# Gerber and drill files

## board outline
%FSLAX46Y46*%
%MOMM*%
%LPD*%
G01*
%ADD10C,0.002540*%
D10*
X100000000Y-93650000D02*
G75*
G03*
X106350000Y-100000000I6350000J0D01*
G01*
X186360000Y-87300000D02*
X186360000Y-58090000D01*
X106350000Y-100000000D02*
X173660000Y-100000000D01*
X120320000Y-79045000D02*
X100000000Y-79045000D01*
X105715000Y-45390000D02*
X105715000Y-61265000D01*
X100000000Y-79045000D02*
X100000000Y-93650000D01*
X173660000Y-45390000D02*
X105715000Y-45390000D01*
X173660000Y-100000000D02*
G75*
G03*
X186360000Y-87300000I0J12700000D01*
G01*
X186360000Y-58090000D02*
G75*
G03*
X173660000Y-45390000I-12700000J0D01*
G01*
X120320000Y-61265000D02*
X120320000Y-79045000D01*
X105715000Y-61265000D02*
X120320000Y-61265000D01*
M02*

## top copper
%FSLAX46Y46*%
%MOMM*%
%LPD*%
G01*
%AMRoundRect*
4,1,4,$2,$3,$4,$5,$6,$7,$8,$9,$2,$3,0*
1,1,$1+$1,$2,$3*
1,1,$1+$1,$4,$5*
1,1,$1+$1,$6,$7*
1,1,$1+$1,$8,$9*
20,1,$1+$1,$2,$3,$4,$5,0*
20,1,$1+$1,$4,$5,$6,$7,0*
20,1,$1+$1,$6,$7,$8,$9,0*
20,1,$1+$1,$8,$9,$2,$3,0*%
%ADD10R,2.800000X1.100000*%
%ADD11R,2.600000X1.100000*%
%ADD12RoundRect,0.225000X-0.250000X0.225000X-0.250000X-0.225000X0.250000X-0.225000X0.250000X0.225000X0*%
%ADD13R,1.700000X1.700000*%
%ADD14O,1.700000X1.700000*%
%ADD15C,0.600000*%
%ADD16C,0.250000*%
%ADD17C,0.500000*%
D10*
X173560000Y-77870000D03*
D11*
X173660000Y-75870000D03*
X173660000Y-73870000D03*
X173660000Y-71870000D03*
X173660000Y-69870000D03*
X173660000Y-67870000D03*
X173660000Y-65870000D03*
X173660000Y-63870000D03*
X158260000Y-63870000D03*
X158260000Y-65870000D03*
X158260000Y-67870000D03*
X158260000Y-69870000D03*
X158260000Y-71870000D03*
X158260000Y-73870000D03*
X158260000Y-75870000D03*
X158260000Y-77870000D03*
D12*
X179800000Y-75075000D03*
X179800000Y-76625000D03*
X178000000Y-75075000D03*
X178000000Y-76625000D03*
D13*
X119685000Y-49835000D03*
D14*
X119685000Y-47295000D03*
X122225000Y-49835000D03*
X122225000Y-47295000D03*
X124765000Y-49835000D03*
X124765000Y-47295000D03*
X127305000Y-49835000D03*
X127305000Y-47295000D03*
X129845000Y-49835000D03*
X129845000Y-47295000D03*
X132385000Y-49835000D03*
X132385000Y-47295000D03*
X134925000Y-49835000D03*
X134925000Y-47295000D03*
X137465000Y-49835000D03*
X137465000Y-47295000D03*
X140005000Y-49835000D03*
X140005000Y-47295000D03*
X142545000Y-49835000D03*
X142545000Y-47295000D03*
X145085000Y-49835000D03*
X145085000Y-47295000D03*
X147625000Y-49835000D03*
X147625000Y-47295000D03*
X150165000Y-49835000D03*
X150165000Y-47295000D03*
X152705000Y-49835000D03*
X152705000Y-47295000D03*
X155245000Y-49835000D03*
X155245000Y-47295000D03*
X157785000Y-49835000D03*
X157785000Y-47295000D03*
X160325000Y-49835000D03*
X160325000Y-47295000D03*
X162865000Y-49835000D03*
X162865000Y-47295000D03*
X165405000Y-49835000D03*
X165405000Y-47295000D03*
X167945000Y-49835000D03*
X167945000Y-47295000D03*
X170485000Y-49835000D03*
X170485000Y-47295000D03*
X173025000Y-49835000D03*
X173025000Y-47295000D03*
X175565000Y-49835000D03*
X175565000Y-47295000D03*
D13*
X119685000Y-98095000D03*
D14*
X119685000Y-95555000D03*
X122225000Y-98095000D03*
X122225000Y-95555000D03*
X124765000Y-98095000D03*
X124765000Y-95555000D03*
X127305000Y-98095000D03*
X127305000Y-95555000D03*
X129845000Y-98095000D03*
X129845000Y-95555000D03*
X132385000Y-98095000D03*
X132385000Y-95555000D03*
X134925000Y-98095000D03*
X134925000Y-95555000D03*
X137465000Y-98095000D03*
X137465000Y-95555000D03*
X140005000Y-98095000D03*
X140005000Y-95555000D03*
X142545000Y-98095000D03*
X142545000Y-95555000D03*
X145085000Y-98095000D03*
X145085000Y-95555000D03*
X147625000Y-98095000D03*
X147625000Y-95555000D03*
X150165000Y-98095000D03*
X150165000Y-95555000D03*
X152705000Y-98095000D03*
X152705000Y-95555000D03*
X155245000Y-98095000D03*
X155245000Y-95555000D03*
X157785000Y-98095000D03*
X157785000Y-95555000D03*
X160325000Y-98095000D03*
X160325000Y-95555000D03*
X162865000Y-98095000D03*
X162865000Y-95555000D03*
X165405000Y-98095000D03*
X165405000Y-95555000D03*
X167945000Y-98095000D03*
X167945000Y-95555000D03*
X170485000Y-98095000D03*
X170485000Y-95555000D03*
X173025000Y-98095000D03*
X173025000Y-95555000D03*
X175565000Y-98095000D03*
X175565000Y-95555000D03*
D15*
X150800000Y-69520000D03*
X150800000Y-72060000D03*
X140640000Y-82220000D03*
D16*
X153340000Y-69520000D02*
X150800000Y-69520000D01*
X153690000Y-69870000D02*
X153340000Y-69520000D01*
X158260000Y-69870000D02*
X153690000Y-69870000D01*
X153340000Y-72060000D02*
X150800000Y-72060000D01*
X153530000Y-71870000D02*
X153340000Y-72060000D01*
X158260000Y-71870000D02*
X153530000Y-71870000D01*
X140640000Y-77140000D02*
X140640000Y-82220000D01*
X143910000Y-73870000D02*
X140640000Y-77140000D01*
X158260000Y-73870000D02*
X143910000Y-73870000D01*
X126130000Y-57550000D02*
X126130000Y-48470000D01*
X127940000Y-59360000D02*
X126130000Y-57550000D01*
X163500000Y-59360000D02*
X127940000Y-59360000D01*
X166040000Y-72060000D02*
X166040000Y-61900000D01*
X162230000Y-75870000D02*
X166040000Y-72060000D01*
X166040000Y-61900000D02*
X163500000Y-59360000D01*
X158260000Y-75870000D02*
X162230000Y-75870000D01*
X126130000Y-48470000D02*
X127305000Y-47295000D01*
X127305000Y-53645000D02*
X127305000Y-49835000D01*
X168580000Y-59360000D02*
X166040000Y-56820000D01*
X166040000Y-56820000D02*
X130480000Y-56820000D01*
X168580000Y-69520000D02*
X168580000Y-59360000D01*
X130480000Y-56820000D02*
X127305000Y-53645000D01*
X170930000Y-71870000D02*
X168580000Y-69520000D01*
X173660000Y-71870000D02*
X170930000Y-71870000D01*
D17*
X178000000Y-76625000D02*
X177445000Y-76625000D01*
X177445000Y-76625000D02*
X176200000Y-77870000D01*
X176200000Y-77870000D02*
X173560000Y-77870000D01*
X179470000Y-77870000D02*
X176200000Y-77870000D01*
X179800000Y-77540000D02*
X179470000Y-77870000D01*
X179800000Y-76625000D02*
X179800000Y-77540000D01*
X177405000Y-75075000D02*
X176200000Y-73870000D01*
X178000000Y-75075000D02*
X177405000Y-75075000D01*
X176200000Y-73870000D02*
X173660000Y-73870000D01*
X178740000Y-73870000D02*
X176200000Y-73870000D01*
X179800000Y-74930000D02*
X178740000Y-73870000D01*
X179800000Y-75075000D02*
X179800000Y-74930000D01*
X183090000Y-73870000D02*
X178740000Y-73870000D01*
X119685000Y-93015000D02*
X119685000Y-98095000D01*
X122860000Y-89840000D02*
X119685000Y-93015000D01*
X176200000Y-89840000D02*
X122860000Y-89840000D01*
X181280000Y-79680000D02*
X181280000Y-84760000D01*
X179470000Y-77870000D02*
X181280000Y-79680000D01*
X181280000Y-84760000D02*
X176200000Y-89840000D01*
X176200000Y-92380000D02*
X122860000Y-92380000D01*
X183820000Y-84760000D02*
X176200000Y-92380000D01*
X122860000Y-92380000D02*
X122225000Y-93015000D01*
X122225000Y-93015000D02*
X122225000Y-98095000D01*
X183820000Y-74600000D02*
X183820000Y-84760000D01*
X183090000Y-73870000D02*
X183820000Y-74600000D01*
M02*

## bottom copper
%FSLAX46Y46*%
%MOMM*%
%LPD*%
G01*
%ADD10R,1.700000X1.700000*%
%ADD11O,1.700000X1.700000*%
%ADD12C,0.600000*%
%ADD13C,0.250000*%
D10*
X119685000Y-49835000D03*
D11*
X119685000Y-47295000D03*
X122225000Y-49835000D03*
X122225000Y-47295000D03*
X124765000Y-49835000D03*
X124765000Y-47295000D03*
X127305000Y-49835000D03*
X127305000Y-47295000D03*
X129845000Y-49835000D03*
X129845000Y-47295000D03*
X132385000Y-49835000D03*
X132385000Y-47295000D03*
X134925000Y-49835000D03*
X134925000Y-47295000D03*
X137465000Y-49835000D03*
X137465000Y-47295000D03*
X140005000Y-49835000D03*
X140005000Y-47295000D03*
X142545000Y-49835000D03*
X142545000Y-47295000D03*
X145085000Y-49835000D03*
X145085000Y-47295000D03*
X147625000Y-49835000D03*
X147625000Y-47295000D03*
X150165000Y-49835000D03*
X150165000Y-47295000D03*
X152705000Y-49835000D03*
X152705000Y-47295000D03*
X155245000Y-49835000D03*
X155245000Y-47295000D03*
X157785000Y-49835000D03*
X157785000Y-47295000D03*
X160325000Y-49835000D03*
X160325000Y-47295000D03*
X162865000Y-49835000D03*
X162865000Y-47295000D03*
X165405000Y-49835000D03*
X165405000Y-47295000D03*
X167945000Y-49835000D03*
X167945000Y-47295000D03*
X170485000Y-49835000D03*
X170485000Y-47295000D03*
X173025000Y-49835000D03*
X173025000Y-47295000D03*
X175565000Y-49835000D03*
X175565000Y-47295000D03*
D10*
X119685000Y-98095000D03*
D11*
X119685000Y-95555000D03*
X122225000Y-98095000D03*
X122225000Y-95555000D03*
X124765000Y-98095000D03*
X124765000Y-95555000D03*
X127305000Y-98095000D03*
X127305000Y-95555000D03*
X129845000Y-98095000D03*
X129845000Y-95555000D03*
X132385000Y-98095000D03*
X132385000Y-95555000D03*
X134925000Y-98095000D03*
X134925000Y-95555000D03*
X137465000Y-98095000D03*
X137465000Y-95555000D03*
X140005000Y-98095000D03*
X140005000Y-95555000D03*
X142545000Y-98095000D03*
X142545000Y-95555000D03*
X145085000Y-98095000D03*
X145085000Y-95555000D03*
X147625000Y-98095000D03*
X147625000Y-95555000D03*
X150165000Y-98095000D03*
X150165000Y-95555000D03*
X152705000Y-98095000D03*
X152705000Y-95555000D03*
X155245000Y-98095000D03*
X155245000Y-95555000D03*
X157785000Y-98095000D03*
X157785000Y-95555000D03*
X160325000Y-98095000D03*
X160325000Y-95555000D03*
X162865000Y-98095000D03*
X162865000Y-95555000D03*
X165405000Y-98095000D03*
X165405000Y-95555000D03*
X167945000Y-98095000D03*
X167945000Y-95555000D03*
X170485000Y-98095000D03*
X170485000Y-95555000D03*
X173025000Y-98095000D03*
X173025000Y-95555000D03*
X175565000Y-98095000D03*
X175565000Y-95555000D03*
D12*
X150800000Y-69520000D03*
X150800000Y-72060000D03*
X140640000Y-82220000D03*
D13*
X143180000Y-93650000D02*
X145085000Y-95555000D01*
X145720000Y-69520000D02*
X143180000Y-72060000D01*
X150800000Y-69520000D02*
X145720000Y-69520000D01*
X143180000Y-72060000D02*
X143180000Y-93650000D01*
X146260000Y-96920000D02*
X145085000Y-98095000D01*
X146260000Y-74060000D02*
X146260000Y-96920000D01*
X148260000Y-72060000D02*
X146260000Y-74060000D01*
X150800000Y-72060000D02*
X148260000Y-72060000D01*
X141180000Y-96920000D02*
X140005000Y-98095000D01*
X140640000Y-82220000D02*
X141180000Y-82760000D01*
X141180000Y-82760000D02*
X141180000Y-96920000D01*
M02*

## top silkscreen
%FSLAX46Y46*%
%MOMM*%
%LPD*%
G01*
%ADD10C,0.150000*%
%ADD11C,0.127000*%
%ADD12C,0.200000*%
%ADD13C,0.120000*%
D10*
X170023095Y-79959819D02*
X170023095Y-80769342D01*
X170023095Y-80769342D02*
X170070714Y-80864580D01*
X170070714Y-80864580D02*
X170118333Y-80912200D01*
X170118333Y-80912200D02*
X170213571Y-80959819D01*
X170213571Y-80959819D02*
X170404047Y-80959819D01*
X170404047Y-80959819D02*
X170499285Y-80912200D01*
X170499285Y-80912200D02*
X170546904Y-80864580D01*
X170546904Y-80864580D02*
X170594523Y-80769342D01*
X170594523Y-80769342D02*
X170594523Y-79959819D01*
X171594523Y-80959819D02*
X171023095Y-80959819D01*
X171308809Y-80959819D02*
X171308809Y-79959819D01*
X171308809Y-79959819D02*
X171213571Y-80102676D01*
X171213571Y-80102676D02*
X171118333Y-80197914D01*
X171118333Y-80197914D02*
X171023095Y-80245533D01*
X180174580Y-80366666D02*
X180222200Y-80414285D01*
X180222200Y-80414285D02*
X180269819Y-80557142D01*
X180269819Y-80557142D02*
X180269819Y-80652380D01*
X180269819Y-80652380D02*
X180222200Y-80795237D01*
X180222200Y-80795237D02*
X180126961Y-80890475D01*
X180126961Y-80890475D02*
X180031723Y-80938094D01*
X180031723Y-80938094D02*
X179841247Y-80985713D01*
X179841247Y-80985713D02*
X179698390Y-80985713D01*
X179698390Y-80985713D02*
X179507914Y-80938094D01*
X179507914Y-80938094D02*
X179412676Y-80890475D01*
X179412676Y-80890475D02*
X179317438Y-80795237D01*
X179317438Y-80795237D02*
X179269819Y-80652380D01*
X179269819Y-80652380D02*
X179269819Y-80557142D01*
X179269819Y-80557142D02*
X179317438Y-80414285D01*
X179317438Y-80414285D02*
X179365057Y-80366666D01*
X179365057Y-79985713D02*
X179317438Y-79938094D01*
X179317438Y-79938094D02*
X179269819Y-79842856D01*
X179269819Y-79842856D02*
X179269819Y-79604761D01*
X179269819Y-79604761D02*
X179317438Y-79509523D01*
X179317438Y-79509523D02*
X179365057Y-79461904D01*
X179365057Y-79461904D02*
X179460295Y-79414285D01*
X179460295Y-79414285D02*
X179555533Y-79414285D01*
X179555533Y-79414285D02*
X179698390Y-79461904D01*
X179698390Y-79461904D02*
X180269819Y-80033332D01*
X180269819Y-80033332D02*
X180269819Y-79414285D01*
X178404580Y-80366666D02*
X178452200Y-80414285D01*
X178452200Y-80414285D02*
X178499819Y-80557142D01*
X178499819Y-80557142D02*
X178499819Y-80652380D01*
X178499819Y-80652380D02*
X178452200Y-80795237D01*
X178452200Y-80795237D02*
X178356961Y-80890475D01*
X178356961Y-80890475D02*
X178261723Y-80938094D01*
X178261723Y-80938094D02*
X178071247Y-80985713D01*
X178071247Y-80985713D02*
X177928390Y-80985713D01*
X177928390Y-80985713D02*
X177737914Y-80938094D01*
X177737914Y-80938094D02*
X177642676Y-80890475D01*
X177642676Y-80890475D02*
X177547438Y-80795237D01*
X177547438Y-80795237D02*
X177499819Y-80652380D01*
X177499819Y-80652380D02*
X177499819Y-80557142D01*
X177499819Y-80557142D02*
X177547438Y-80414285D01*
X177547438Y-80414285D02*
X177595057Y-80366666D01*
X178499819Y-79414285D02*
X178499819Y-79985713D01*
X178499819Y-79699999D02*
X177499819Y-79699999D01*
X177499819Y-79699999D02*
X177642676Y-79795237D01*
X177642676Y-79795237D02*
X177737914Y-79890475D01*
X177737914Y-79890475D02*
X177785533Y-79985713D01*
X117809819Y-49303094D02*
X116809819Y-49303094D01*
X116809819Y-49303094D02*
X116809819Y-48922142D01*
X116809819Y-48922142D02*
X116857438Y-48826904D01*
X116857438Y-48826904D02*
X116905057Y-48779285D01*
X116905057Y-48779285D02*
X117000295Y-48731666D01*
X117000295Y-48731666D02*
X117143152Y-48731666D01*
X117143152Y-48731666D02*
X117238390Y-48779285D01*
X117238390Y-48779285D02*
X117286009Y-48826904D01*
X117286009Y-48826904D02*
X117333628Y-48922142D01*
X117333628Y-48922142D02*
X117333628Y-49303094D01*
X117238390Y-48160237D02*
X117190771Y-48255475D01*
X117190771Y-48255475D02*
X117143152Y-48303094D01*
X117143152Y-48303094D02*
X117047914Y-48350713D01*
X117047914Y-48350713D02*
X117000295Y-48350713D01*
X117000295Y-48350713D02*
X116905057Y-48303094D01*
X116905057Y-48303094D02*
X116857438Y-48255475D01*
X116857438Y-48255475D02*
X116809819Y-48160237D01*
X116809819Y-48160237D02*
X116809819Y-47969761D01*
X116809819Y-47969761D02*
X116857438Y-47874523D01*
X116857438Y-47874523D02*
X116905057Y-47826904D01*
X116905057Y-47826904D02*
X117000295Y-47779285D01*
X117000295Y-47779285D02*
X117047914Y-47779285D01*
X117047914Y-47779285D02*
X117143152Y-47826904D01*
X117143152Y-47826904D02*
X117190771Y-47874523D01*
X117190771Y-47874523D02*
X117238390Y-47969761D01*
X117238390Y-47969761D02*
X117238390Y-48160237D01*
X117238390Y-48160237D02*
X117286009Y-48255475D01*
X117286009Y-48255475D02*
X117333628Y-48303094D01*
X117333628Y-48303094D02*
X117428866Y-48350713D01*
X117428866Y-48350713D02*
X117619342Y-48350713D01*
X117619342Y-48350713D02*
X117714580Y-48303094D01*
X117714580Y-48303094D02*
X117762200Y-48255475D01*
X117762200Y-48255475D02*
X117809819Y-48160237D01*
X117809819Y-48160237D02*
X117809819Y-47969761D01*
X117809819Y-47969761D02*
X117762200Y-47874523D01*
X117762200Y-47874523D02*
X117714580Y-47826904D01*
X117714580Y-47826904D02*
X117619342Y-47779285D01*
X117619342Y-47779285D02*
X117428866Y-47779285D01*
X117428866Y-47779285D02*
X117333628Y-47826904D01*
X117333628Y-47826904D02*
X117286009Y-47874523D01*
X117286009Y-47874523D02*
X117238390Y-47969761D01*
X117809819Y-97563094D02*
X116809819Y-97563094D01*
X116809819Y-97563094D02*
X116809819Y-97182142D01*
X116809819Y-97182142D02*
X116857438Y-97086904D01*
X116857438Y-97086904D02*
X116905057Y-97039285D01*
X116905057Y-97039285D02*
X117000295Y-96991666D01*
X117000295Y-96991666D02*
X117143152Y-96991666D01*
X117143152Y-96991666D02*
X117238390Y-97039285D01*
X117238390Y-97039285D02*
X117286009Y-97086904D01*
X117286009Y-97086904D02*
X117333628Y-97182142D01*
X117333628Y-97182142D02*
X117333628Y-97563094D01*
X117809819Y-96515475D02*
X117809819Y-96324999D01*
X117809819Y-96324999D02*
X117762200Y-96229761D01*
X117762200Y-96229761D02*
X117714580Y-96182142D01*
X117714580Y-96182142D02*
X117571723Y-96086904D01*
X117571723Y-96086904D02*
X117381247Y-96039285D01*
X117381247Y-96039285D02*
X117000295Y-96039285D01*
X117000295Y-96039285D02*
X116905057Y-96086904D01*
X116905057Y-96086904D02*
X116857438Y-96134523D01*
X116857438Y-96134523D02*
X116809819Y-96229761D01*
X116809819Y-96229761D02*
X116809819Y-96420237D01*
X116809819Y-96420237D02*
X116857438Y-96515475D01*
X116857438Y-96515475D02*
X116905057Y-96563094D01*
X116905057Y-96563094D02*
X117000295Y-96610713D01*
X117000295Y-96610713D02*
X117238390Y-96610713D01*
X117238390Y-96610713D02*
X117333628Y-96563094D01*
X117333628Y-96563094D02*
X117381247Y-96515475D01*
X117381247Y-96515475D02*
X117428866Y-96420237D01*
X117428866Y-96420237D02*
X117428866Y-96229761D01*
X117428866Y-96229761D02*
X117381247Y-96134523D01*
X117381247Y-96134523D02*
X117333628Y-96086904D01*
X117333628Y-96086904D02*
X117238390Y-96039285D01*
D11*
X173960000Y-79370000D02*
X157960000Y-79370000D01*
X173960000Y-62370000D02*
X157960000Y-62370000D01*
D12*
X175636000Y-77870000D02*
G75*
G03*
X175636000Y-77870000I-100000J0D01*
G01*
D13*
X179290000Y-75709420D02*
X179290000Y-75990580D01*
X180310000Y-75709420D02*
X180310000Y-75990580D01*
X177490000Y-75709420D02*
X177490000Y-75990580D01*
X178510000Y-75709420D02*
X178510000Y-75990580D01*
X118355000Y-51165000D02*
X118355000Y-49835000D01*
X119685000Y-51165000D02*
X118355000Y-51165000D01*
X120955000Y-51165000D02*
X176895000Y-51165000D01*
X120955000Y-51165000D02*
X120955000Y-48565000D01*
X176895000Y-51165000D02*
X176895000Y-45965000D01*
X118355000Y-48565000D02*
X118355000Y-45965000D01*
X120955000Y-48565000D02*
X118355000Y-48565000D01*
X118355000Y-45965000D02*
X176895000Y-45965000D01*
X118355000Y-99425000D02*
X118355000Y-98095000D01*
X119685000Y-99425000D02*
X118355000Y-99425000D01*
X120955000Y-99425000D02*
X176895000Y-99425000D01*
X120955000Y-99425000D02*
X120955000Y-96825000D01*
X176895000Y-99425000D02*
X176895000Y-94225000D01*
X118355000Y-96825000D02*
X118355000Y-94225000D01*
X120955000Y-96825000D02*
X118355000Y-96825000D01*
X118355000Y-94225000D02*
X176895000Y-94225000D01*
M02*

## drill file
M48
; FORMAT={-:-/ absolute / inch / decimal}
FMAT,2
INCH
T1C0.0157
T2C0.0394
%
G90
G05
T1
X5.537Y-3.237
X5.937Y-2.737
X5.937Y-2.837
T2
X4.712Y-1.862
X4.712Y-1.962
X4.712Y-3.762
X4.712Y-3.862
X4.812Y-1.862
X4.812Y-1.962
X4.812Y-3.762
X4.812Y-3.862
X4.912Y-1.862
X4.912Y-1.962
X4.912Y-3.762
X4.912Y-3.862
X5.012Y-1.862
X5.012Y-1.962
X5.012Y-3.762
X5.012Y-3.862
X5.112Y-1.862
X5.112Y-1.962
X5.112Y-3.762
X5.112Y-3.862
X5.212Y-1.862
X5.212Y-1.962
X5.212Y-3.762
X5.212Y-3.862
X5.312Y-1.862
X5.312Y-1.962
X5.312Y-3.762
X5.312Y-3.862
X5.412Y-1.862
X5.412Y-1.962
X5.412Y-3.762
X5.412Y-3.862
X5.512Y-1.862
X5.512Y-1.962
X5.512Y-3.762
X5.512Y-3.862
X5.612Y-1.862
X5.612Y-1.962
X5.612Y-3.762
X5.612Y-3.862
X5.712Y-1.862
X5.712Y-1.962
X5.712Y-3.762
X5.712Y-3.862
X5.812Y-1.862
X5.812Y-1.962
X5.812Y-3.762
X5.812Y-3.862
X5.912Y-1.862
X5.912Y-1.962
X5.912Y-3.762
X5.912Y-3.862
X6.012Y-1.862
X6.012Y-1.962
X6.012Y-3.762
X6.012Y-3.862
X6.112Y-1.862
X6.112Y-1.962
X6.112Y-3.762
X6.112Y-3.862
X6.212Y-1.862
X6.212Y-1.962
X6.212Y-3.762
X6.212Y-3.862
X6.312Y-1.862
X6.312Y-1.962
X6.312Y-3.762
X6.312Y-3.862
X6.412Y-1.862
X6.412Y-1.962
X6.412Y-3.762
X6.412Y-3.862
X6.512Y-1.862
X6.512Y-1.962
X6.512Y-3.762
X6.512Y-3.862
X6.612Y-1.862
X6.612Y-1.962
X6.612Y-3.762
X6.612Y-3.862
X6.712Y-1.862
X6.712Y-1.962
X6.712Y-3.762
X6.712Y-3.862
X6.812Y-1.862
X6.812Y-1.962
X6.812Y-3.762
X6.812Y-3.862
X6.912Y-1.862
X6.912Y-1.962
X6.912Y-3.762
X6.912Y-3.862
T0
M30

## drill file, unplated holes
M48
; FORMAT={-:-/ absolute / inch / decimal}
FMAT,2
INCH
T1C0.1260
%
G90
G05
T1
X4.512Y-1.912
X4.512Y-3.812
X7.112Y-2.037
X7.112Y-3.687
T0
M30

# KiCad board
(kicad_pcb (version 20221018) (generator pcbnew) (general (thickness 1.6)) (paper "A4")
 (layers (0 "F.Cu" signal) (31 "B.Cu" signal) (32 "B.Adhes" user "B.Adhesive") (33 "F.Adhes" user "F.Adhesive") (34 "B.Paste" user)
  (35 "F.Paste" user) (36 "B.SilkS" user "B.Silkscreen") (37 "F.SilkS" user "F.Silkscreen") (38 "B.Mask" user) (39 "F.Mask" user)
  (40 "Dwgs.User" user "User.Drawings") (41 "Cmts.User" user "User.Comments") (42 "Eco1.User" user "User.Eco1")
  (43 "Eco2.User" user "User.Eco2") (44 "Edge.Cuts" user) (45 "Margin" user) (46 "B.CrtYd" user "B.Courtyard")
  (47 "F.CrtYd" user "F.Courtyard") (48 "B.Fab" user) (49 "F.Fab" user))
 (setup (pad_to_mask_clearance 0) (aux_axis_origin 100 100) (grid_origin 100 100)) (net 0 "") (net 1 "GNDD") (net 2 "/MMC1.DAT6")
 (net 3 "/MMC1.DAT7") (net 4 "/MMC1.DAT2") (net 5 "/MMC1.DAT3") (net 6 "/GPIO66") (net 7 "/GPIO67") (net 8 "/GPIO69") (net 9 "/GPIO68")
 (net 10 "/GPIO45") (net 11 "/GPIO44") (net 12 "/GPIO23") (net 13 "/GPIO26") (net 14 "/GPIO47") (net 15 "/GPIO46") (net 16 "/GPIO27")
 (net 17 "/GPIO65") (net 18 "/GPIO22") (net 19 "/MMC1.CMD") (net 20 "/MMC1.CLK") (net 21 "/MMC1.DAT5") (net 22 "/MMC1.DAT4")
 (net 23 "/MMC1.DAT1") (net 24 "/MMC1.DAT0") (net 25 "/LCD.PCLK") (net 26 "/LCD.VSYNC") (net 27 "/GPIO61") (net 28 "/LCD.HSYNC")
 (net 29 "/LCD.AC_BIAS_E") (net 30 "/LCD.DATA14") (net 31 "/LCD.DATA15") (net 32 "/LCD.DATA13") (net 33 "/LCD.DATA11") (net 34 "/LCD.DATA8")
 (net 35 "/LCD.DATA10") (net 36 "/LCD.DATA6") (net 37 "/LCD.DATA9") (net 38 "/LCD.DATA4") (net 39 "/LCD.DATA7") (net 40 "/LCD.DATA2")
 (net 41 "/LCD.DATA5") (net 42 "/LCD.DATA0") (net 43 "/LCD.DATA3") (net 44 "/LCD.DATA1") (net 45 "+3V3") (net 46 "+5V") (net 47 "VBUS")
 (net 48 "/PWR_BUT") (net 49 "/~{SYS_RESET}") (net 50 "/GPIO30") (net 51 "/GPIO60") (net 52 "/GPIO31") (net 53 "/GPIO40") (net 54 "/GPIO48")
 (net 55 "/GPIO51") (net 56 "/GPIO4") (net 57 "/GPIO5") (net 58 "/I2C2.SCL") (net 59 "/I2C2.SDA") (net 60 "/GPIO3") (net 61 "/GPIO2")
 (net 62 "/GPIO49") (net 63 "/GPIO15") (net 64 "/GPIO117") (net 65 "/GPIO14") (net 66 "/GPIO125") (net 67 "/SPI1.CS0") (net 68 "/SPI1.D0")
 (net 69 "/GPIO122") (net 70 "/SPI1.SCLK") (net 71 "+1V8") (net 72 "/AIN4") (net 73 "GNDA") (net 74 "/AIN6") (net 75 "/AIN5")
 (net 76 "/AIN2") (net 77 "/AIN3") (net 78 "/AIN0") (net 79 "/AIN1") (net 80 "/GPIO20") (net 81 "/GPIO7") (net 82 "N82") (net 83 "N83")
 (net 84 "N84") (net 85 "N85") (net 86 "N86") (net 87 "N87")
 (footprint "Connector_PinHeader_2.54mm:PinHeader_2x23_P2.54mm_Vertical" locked (layer "F.Cu") (at 119.685 49.835 90)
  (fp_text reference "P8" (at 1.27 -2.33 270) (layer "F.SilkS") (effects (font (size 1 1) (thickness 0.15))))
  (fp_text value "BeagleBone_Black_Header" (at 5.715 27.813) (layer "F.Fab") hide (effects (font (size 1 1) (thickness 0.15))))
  (fp_line (start -1.33 -1.33) (end 0 -1.33) (stroke (width 0.12) (type solid)) (layer "F.SilkS"))
  (fp_line (start -1.33 0) (end -1.33 -1.33) (stroke (width 0.12) (type solid)) (layer "F.SilkS"))
  (fp_line (start -1.33 1.27) (end -1.33 57.21) (stroke (width 0.12) (type solid)) (layer "F.SilkS"))
  (fp_line (start -1.33 1.27) (end 1.27 1.27) (stroke (width 0.12) (type solid)) (layer "F.SilkS"))
  (fp_line (start -1.33 57.21) (end 3.87 57.21) (stroke (width 0.12) (type solid)) (layer "F.SilkS"))
  (fp_line (start 1.27 -1.33) (end 3.87 -1.33) (stroke (width 0.12) (type solid)) (layer "F.SilkS"))
  (fp_line (start 1.27 1.27) (end 1.27 -1.33) (stroke (width 0.12) (type solid)) (layer "F.SilkS"))
  (fp_line (start 3.87 -1.33) (end 3.87 57.21) (stroke (width 0.12) (type solid)) (layer "F.SilkS"))
  (pad "1" thru_hole rect locked (at 0 0 90) (size 1.7 1.7) (drill 1) (layers "*.Cu" "*.Mask") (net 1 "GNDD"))
  (pad "2" thru_hole oval locked (at 2.54 0 90) (size 1.7 1.7) (drill 1) (layers "*.Cu" "*.Mask") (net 1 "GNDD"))
  (pad "3" thru_hole oval locked (at 0 2.54 90) (size 1.7 1.7) (drill 1) (layers "*.Cu" "*.Mask") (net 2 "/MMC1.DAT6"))
  (pad "4" thru_hole oval locked (at 2.54 2.54 90) (size 1.7 1.7) (drill 1) (layers "*.Cu" "*.Mask") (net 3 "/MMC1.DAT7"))
  (pad "5" thru_hole oval locked (at 0 5.08 90) (size 1.7 1.7) (drill 1) (layers "*.Cu" "*.Mask") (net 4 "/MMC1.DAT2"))
  (pad "6" thru_hole oval locked (at 2.54 5.08 90) (size 1.7 1.7) (drill 1) (layers "*.Cu" "*.Mask") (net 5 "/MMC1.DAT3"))
  (pad "7" thru_hole oval locked (at 0 7.62 90) (size 1.7 1.7) (drill 1) (layers "*.Cu" "*.Mask") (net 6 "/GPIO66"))
  (pad "8" thru_hole oval locked (at 2.54 7.62 90) (size 1.7 1.7) (drill 1) (layers "*.Cu" "*.Mask") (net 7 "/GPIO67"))
  (pad "9" thru_hole oval locked (at 0 10.16 90) (size 1.7 1.7) (drill 1) (layers "*.Cu" "*.Mask") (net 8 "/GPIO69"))
  (pad "10" thru_hole oval locked (at 2.54 10.16 90) (size 1.7 1.7) (drill 1) (layers "*.Cu" "*.Mask") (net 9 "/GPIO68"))
  (pad "11" thru_hole oval locked (at 0 12.7 90) (size 1.7 1.7) (drill 1) (layers "*.Cu" "*.Mask") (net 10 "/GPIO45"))
  (pad "12" thru_hole oval locked (at 2.54 12.7 90) (size 1.7 1.7) (drill 1) (layers "*.Cu" "*.Mask") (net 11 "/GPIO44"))
  (pad "13" thru_hole oval locked (at 0 15.24 90) (size 1.7 1.7) (drill 1) (layers "*.Cu" "*.Mask") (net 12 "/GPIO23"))
  (pad "14" thru_hole oval locked (at 2.54 15.24 90) (size 1.7 1.7) (drill 1) (layers "*.Cu" "*.Mask") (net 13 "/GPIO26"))
  (pad "15" thru_hole oval locked (at 0 17.78 90) (size 1.7 1.7) (drill 1) (layers "*.Cu" "*.Mask") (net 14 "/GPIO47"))
  (pad "16" thru_hole oval locked (at 2.54 17.78 90) (size 1.7 1.7) (drill 1) (layers "*.Cu" "*.Mask") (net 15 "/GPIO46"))
  (pad "17" thru_hole oval locked (at 0 20.32 90) (size 1.7 1.7) (drill 1) (layers "*.Cu" "*.Mask") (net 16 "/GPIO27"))
  (pad "18" thru_hole oval locked (at 2.54 20.32 90) (size 1.7 1.7) (drill 1) (layers "*.Cu" "*.Mask") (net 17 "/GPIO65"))
  (pad "19" thru_hole oval locked (at 0 22.86 90) (size 1.7 1.7) (drill 1) (layers "*.Cu" "*.Mask") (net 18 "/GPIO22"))
  (pad "20" thru_hole oval locked (at 2.54 22.86 90) (size 1.7 1.7) (drill 1) (layers "*.Cu" "*.Mask") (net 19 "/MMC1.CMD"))
  (pad "21" thru_hole oval locked (at 0 25.4 90) (size 1.7 1.7) (drill 1) (layers "*.Cu" "*.Mask") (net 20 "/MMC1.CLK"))
  (pad "22" thru_hole oval locked (at 2.54 25.4 90) (size 1.7 1.7) (drill 1) (layers "*.Cu" "*.Mask") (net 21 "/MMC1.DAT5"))
  (pad "23" thru_hole oval locked (at 0 27.94 90) (size 1.7 1.7) (drill 1) (layers "*.Cu" "*.Mask") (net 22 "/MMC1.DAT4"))
  (pad "24" thru_hole oval locked (at 2.54 27.94 90) (size 1.7 1.7) (drill 1) (layers "*.Cu" "*.Mask") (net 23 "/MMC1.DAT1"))
  (pad "25" thru_hole oval locked (at 0 30.48 90) (size 1.7 1.7) (drill 1) (layers "*.Cu" "*.Mask") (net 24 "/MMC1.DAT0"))
  (pad "26" thru_hole oval locked (at 2.54 30.48 90) (size 1.7 1.7) (drill 1) (layers "*.Cu" "*.Mask") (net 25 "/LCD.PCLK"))
  (pad "27" thru_hole oval locked (at 0 33.02 90) (size 1.7 1.7) (drill 1) (layers "*.Cu" "*.Mask") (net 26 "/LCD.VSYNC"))
  (pad "28" thru_hole oval locked (at 2.54 33.02 90) (size 1.7 1.7) (drill 1) (layers "*.Cu" "*.Mask") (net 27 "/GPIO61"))
  (pad "29" thru_hole oval locked (at 0 35.56 90) (size 1.7 1.7) (drill 1) (layers "*.Cu" "*.Mask") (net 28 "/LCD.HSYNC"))
  (pad "30" thru_hole oval locked (at 2.54 35.56 90) (size 1.7 1.7) (drill 1) (layers "*.Cu" "*.Mask") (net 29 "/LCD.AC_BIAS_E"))
  (pad "31" thru_hole oval locked (at 0 38.1 90) (size 1.7 1.7) (drill 1) (layers "*.Cu" "*.Mask") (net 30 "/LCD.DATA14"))
  (pad "32" thru_hole oval locked (at 2.54 38.1 90) (size 1.7 1.7) (drill 1) (layers "*.Cu" "*.Mask") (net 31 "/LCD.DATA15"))
  (pad "33" thru_hole oval locked (at 0 40.64 90) (size 1.7 1.7) (drill 1) (layers "*.Cu" "*.Mask") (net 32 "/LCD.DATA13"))
  (pad "34" thru_hole oval locked (at 2.54 40.64 90) (size 1.7 1.7) (drill 1) (layers "*.Cu" "*.Mask") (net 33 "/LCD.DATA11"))
  (pad "35" thru_hole oval locked (at 0 43.18 90) (size 1.7 1.7) (drill 1) (layers "*.Cu" "*.Mask") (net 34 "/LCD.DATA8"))
  (pad "36" thru_hole oval locked (at 2.54 43.18 90) (size 1.7 1.7) (drill 1) (layers "*.Cu" "*.Mask") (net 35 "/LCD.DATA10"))
  (pad "37" thru_hole oval locked (at 0 45.72 90) (size 1.7 1.7) (drill 1) (layers "*.Cu" "*.Mask") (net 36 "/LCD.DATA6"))
  (pad "38" thru_hole oval locked (at 2.54 45.72 90) (size 1.7 1.7) (drill 1) (layers "*.Cu" "*.Mask") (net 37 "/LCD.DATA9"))
  (pad "39" thru_hole oval locked (at 0 48.26 90) (size 1.7 1.7) (drill 1) (layers "*.Cu" "*.Mask") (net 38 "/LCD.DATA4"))
  (pad "40" thru_hole oval locked (at 2.54 48.26 90) (size 1.7 1.7) (drill 1) (layers "*.Cu" "*.Mask") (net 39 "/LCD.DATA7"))
  (pad "41" thru_hole oval locked (at 0 50.8 90) (size 1.7 1.7) (drill 1) (layers "*.Cu" "*.Mask") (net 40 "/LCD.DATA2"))
  (pad "42" thru_hole oval locked (at 2.54 50.8 90) (size 1.7 1.7) (drill 1) (layers "*.Cu" "*.Mask") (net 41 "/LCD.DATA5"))
  (pad "43" thru_hole oval locked (at 0 53.34 90) (size 1.7 1.7) (drill 1) (layers "*.Cu" "*.Mask") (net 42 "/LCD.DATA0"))
  (pad "44" thru_hole oval locked (at 2.54 53.34 90) (size 1.7 1.7) (drill 1) (layers "*.Cu" "*.Mask") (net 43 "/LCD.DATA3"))
  (pad "45" thru_hole oval locked (at 0 55.88 90) (size 1.7 1.7) (drill 1) (layers "*.Cu" "*.Mask") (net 1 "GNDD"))
  (pad "46" thru_hole oval locked (at 2.54 55.88 90) (size 1.7 1.7) (drill 1) (layers "*.Cu" "*.Mask") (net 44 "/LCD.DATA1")))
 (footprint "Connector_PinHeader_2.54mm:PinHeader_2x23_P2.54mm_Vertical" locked (layer "F.Cu") (at 119.685 98.095 90)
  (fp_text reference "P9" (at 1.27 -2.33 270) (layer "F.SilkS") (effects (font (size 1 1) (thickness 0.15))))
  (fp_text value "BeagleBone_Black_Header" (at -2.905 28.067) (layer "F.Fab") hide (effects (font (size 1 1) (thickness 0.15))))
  (fp_line (start -1.33 -1.33) (end 0 -1.33) (stroke (width 0.12) (type solid)) (layer "F.SilkS"))
  (fp_line (start -1.33 0) (end -1.33 -1.33) (stroke (width 0.12) (type solid)) (layer "F.SilkS"))
  (fp_line (start -1.33 1.27) (end -1.33 57.21) (stroke (width 0.12) (type solid)) (layer "F.SilkS"))
  (fp_line (start -1.33 1.27) (end 1.27 1.27) (stroke (width 0.12) (type solid)) (layer "F.SilkS"))
  (fp_line (start -1.33 57.21) (end 3.87 57.21) (stroke (width 0.12) (type solid)) (layer "F.SilkS"))
  (fp_line (start 1.27 -1.33) (end 3.87 -1.33) (stroke (width 0.12) (type solid)) (layer "F.SilkS"))
  (fp_line (start 1.27 1.27) (end 1.27 -1.33) (stroke (width 0.12) (type solid)) (layer "F.SilkS"))
  (fp_line (start 3.87 -1.33) (end 3.87 57.21) (stroke (width 0.12) (type solid)) (layer "F.SilkS"))
  (pad "1" thru_hole rect locked (at 0 0 90) (size 1.7 1.7) (drill 1) (layers "*.Cu" "*.Mask") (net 1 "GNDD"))
  (pad "2" thru_hole oval locked (at 2.54 0 90) (size 1.7 1.7) (drill 1) (layers "*.Cu" "*.Mask") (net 1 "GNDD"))
  (pad "3" thru_hole oval locked (at 0 2.54 90) (size 1.7 1.7) (drill 1) (layers "*.Cu" "*.Mask") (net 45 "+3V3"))
  (pad "4" thru_hole oval locked (at 2.54 2.54 90) (size 1.7 1.7) (drill 1) (layers "*.Cu" "*.Mask") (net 45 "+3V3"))
  (pad "5" thru_hole oval locked (at 0 5.08 90) (size 1.7 1.7) (drill 1) (layers "*.Cu" "*.Mask") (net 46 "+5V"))
  (pad "6" thru_hole oval locked (at 2.54 5.08 90) (size 1.7 1.7) (drill 1) (layers "*.Cu" "*.Mask") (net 46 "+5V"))
  (pad "7" thru_hole oval locked (at 0 7.62 90) (size 1.7 1.7) (drill 1) (layers "*.Cu" "*.Mask") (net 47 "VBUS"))
  (pad "8" thru_hole oval locked (at 2.54 7.62 90) (size 1.7 1.7) (drill 1) (layers "*.Cu" "*.Mask") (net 47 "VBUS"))
  (pad "9" thru_hole oval locked (at 0 10.16 90) (size 1.7 1.7) (drill 1) (layers "*.Cu" "*.Mask") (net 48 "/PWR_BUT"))
  (pad "10" thru_hole oval locked (at 2.54 10.16 90) (size 1.7 1.7) (drill 1) (layers "*.Cu" "*.Mask") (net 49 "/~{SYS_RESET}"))
  (pad "11" thru_hole oval locked (at 0 12.7 90) (size 1.7 1.7) (drill 1) (layers "*.Cu" "*.Mask") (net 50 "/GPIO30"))
  (pad "12" thru_hole oval locked (at 2.54 12.7 90) (size 1.7 1.7) (drill 1) (layers "*.Cu" "*.Mask") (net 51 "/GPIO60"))
  (pad "13" thru_hole oval locked (at 0 15.24 90) (size 1.7 1.7) (drill 1) (layers "*.Cu" "*.Mask") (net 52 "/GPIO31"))
  (pad "14" thru_hole oval locked (at 2.54 15.24 90) (size 1.7 1.7) (drill 1) (layers "*.Cu" "*.Mask") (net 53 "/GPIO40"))
  (pad "15" thru_hole oval locked (at 0 17.78 90) (size 1.7 1.7) (drill 1) (layers "*.Cu" "*.Mask") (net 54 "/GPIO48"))
  (pad "16" thru_hole oval locked (at 2.54 17.78 90) (size 1.7 1.7) (drill 1) (layers "*.Cu" "*.Mask") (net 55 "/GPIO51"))
  (pad "17" thru_hole oval locked (at 0 20.32 90) (size 1.7 1.7) (drill 1) (layers "*.Cu" "*.Mask") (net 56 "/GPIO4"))
  (pad "18" thru_hole oval locked (at 2.54 20.32 90) (size 1.7 1.7) (drill 1) (layers "*.Cu" "*.Mask") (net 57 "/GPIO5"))
  (pad "19" thru_hole oval locked (at 0 22.86 90) (size 1.7 1.7) (drill 1) (layers "*.Cu" "*.Mask") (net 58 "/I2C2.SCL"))
  (pad "20" thru_hole oval locked (at 2.54 22.86 90) (size 1.7 1.7) (drill 1) (layers "*.Cu" "*.Mask") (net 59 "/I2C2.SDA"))
  (pad "21" thru_hole oval locked (at 0 25.4 90) (size 1.7 1.7) (drill 1) (layers "*.Cu" "*.Mask") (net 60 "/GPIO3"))
  (pad "22" thru_hole oval locked (at 2.54 25.4 90) (size 1.7 1.7) (drill 1) (layers "*.Cu" "*.Mask") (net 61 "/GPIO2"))
  (pad "23" thru_hole oval locked (at 0 27.94 90) (size 1.7 1.7) (drill 1) (layers "*.Cu" "*.Mask") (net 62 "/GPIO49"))
  (pad "24" thru_hole oval locked (at 2.54 27.94 90) (size 1.7 1.7) (drill 1) (layers "*.Cu" "*.Mask") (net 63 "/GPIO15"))
  (pad "25" thru_hole oval locked (at 0 30.48 90) (size 1.7 1.7) (drill 1) (layers "*.Cu" "*.Mask") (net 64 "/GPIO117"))
  (pad "26" thru_hole oval locked (at 2.54 30.48 90) (size 1.7 1.7) (drill 1) (layers "*.Cu" "*.Mask") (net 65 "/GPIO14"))
  (pad "27" thru_hole oval locked (at 0 33.02 90) (size 1.7 1.7) (drill 1) (layers "*.Cu" "*.Mask") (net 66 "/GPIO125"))
  (pad "28" thru_hole oval locked (at 2.54 33.02 90) (size 1.7 1.7) (drill 1) (layers "*.Cu" "*.Mask") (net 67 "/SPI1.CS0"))
  (pad "29" thru_hole oval locked (at 0 35.56 90) (size 1.7 1.7) (drill 1) (layers "*.Cu" "*.Mask") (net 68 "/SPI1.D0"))
  (pad "30" thru_hole oval locked (at 2.54 35.56 90) (size 1.7 1.7) (drill 1) (layers "*.Cu" "*.Mask") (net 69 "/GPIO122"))
  (pad "31" thru_hole oval locked (at 0 38.1 90) (size 1.7 1.7) (drill 1) (layers "*.Cu" "*.Mask") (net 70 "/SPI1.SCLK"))
  (pad "32" thru_hole oval locked (at 2.54 38.1 90) (size 1.7 1.7) (drill 1) (layers "*.Cu" "*.Mask") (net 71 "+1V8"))
  (pad "33" thru_hole oval locked (at 0 40.64 90) (size 1.7 1.7) (drill 1) (layers "*.Cu" "*.Mask") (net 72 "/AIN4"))
  (pad "34" thru_hole oval locked (at 2.54 40.64 90) (size 1.7 1.7) (drill 1) (layers "*.Cu" "*.Mask") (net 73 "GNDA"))
  (pad "35" thru_hole oval locked (at 0 43.18 90) (size 1.7 1.7) (drill 1) (layers "*.Cu" "*.Mask") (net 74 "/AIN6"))
  (pad "36" thru_hole oval locked (at 2.54 43.18 90) (size 1.7 1.7) (drill 1) (layers "*.Cu" "*.Mask") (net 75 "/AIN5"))
  (pad "37" thru_hole oval locked (at 0 45.72 90) (size 1.7 1.7) (drill 1) (layers "*.Cu" "*.Mask") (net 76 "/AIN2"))
  (pad "38" thru_hole oval locked (at 2.54 45.72 90) (size 1.7 1.7) (drill 1) (layers "*.Cu" "*.Mask") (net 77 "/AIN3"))
  (pad "39" thru_hole oval locked (at 0 48.26 90) (size 1.7 1.7) (drill 1) (layers "*.Cu" "*.Mask") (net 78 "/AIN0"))
  (pad "40" thru_hole oval locked (at 2.54 48.26 90) (size 1.7 1.7) (drill 1) (layers "*.Cu" "*.Mask") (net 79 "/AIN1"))
  (pad "41" thru_hole oval locked (at 0 50.8 90) (size 1.7 1.7) (drill 1) (layers "*.Cu" "*.Mask") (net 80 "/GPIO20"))
  (pad "42" thru_hole oval locked (at 2.54 50.8 90) (size 1.7 1.7) (drill 1) (layers "*.Cu" "*.Mask") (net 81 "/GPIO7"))
  (pad "43" thru_hole oval locked (at 0 53.34 90) (size 1.7 1.7) (drill 1) (layers "*.Cu" "*.Mask") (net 1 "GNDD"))
  (pad "44" thru_hole oval locked (at 2.54 53.34 90) (size 1.7 1.7) (drill 1) (layers "*.Cu" "*.Mask") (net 1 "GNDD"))
  (pad "45" thru_hole oval locked (at 0 55.88 90) (size 1.7 1.7) (drill 1) (layers "*.Cu" "*.Mask") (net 1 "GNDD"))
  (pad "46" thru_hole oval locked (at 2.54 55.88 90) (size 1.7 1.7) (drill 1) (layers "*.Cu" "*.Mask") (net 1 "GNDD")))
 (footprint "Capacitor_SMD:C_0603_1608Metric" (layer "F.Cu") (at 178 75.85 -90)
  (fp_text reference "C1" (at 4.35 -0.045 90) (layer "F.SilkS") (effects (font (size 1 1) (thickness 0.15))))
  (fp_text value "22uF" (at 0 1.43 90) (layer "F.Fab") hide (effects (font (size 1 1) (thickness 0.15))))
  (fp_line (start -0.14058 -0.51) (end 0.14058 -0.51) (stroke (width 0.12) (type solid)) (layer "F.SilkS"))
  (fp_line (start -0.14058 0.51) (end 0.14058 0.51) (stroke (width 0.12) (type solid)) (layer "F.SilkS"))
  (pad "1" smd roundrect (at -0.775 0 270) (size 0.9 0.95) (layers "F.Cu" "F.Paste" "F.Mask") (roundrect_rratio 0.25) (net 45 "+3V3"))
  (pad "2" smd roundrect (at 0.775 0 270) (size 0.9 0.95) (layers "F.Cu" "F.Paste" "F.Mask") (roundrect_rratio 0.25) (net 1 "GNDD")))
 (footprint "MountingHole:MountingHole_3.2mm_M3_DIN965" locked (layer "F.Cu") (at 180.645 51.74)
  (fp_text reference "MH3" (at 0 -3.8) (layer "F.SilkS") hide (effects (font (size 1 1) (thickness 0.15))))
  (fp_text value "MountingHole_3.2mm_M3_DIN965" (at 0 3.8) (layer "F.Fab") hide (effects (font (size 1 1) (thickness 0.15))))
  (pad "" np_thru_hole circle locked (at 0 0) (size 3.2 3.2) (drill 3.2) (layers "*.Cu" "*.Mask")))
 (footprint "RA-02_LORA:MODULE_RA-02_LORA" (layer "F.Cu") (at 165.96 70.87 180)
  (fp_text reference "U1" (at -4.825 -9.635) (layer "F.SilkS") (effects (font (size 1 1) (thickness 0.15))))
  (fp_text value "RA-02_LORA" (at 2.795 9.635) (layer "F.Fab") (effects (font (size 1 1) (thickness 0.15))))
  (fp_line (start -8 -8.5) (end 8 -8.5) (stroke (width 0.127) (type solid)) (layer "F.SilkS"))
  (fp_line (start -8 8.5) (end 8 8.5) (stroke (width 0.127) (type solid)) (layer "F.SilkS"))
  (fp_circle (center -9.576 -7) (end -9.476 -7) (stroke (width 0.2) (type solid)) (fill none) (layer "F.SilkS"))
  (pad "1" smd rect (at -7.6 -7 180) (size 2.8 1.1) (layers "F.Cu" "F.Paste" "F.Mask") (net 1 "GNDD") (solder_mask_margin 0.102))
  (pad "2" smd rect (at -7.7 -5 180) (size 2.6 1.1) (layers "F.Cu" "F.Paste" "F.Mask") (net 1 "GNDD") (solder_mask_margin 0.102))
  (pad "3" smd rect (at -7.7 -3 180) (size 2.6 1.1) (layers "F.Cu" "F.Paste" "F.Mask") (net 45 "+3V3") (solder_mask_margin 0.102))
  (pad "4" smd rect (at -7.7 -1 180) (size 2.6 1.1) (layers "F.Cu" "F.Paste" "F.Mask") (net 6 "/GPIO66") (solder_mask_margin 0.102))
  (pad "5" smd rect (at -7.7 1 180) (size 2.6 1.1) (layers "F.Cu" "F.Paste" "F.Mask") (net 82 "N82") (solder_mask_margin 0.102))
  (pad "6" smd rect (at -7.7 3 180) (size 2.6 1.1) (layers "F.Cu" "F.Paste" "F.Mask") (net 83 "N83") (solder_mask_margin 0.102))
  (pad "7" smd rect (at -7.7 5 180) (size 2.6 1.1) (layers "F.Cu" "F.Paste" "F.Mask") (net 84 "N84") (solder_mask_margin 0.102))
  (pad "8" smd rect (at -7.7 7 180) (size 2.6 1.1) (layers "F.Cu" "F.Paste" "F.Mask") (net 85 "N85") (solder_mask_margin 0.102))
  (pad "9" smd rect (at 7.7 7) (size 2.6 1.1) (layers "F.Cu" "F.Paste" "F.Mask") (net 1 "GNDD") (solder_mask_margin 0.102))
  (pad "10" smd rect (at 7.7 5) (size 2.6 1.1) (layers "F.Cu" "F.Paste" "F.Mask") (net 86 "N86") (solder_mask_margin 0.102))
  (pad "11" smd rect (at 7.7 3) (size 2.6 1.1) (layers "F.Cu" "F.Paste" "F.Mask") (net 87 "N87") (solder_mask_margin 0.102))
  (pad "12" smd rect (at 7.7 1) (size 2.6 1.1) (layers "F.Cu" "F.Paste" "F.Mask") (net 61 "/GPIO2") (solder_mask_margin 0.102))
  (pad "13" smd rect (at 7.7 -1) (size 2.6 1.1) (layers "F.Cu" "F.Paste" "F.Mask") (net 60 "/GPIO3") (solder_mask_margin 0.102))
  (pad "14" smd rect (at 7.7 -3) (size 2.6 1.1) (layers "F.Cu" "F.Paste" "F.Mask") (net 56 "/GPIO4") (solder_mask_margin 0.102))
  (pad "15" smd rect (at 7.7 -5) (size 2.6 1.1) (layers "F.Cu" "F.Paste" "F.Mask") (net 7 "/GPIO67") (solder_mask_margin 0.102))
  (pad "16" smd rect (at 7.7 -7) (size 2.6 1.1) (layers "F.Cu" "F.Paste" "F.Mask") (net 1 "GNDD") (solder_mask_margin 0.102)))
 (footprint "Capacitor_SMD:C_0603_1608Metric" (layer "F.Cu") (at 179.8 75.85 -90)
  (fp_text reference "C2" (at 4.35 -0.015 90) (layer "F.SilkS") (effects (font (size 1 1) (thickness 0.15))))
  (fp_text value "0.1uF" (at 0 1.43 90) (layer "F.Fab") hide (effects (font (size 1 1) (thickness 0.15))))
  (fp_line (start -0.14058 -0.51) (end 0.14058 -0.51) (stroke (width 0.12) (type solid)) (layer "F.SilkS"))
  (fp_line (start -0.14058 0.51) (end 0.14058 0.51) (stroke (width 0.12) (type solid)) (layer "F.SilkS"))
  (pad "1" smd roundrect (at -0.775 0 270) (size 0.9 0.95) (layers "F.Cu" "F.Paste" "F.Mask") (roundrect_rratio 0.25) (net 45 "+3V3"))
  (pad "2" smd roundrect (at 0.775 0 270) (size 0.9 0.95) (layers "F.Cu" "F.Paste" "F.Mask") (roundrect_rratio 0.25) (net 1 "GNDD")))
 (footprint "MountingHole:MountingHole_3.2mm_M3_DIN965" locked (layer "F.Cu") (at 180.645 93.65)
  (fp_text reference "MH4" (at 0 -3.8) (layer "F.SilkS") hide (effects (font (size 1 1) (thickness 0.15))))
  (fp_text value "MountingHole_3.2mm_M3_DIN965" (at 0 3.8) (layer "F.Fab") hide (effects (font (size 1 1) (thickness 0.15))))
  (pad "" np_thru_hole circle locked (at 0 0) (size 3.2 3.2) (drill 3.2) (layers "*.Cu" "*.Mask")))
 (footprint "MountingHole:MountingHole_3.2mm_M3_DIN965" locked (layer "F.Cu") (at 114.605 48.565)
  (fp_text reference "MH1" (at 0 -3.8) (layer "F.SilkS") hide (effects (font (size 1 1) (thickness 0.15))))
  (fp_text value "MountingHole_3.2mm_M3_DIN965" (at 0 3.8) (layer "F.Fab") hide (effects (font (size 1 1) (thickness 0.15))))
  (pad "" np_thru_hole circle locked (at 0 0) (size 3.2 3.2) (drill 3.2) (layers "*.Cu" "*.Mask")))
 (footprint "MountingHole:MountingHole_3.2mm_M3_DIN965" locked (layer "F.Cu") (at 114.605 96.825)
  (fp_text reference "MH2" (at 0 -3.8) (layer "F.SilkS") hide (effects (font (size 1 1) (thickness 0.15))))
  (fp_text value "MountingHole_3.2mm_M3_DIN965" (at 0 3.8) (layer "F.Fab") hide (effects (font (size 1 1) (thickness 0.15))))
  (pad "" np_thru_hole circle locked (at 0 0) (size 3.2 3.2) (drill 3.2) (layers "*.Cu" "*.Mask")))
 (gr_arc locked (start 106.35 100) (mid 101.859872 98.140128) (end 100 93.65) (stroke (width 0.00254) (type solid)) (layer "Edge.Cuts"))
 (gr_line locked (start 186.36 87.3) (end 186.36 58.09) (stroke (width 0.00254) (type solid)) (layer "Edge.Cuts"))
 (gr_line locked (start 106.35 100) (end 173.66 100) (stroke (width 0.00254) (type solid)) (layer "Edge.Cuts"))
 (gr_line locked (start 120.32 79.045) (end 100 79.045) (stroke (width 0.00254) (type solid)) (layer "Edge.Cuts"))
 (gr_line locked (start 105.715 45.39) (end 105.715 61.265) (stroke (width 0.00254) (type solid)) (layer "Edge.Cuts"))
 (gr_line locked (start 100 79.045) (end 100 93.65) (stroke (width 0.00254) (type solid)) (layer "Edge.Cuts"))
 (gr_line locked (start 173.66 45.39) (end 105.715 45.39) (stroke (width 0.00254) (type solid)) (layer "Edge.Cuts"))
 (gr_arc locked (start 186.36 87.3) (mid 182.640256 96.280256) (end 173.66 100) (stroke (width 0.00254) (type solid)) (layer "Edge.Cuts"))
 (gr_arc locked (start 173.66 45.39) (mid 182.640256 49.109744) (end 186.36 58.09) (stroke (width 0.00254) (type solid)) (layer "Edge.Cuts"))
 (gr_line locked (start 120.32 61.265) (end 120.32 79.045) (stroke (width 0.00254) (type solid)) (layer "Edge.Cuts"))
 (gr_line locked (start 105.715 61.265) (end 120.32 61.265) (stroke (width 0.00254) (type solid)) (layer "Edge.Cuts"))
 (segment (start 130.48 56.82) (end 127.305 53.645) (width 0.25) (layer "F.Cu") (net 6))
 (segment (start 168.58 69.52) (end 168.58 59.36) (width 0.25) (layer "F.Cu") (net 6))
 (segment (start 166.04 56.82) (end 130.48 56.82) (width 0.25) (layer "F.Cu") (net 6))
 (segment (start 168.58 59.36) (end 166.04 56.82) (width 0.25) (layer "F.Cu") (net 6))
 (segment (start 170.93 71.87) (end 168.58 69.52) (width 0.25) (layer "F.Cu") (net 6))
 (segment (start 173.66 71.87) (end 170.93 71.87) (width 0.25) (layer "F.Cu") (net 6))
 (segment (start 127.305 53.645) (end 127.305 49.835) (width 0.25) (layer "F.Cu") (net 6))
 (segment (start 126.13 57.55) (end 126.13 48.47) (width 0.25) (layer "F.Cu") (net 7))
 (segment (start 166.04 72.06) (end 166.04 61.9) (width 0.25) (layer "F.Cu") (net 7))
 (segment (start 127.94 59.36) (end 126.13 57.55) (width 0.25) (layer "F.Cu") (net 7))
 (segment (start 126.13 48.47) (end 127.305 47.295) (width 0.25) (layer "F.Cu") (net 7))
 (segment (start 158.26 75.87) (end 162.23 75.87) (width 0.25) (layer "F.Cu") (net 7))
 (segment (start 163.5 59.36) (end 127.94 59.36) (width 0.25) (layer "F.Cu") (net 7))
 (segment (start 166.04 61.9) (end 163.5 59.36) (width 0.25) (layer "F.Cu") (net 7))
 (segment (start 162.23 75.87) (end 166.04 72.06) (width 0.25) (layer "F.Cu") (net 7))
 (segment (start 181.28 84.76) (end 176.2 89.84) (width 0.5) (layer "F.Cu") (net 1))
 (segment (start 179.47 77.87) (end 181.28 79.68) (width 0.5) (layer "F.Cu") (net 1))
 (segment (start 122.86 89.84) (end 119.685 93.015) (width 0.5) (layer "F.Cu") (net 1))
 (segment (start 179.47 77.87) (end 176.2 77.87) (width 0.5) (layer "F.Cu") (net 1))
 (segment (start 181.28 79.68) (end 181.28 84.76) (width 0.5) (layer "F.Cu") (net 1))
 (segment (start 119.685 93.015) (end 119.685 98.095) (width 0.5) (layer "F.Cu") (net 1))
 (segment (start 176.2 77.87) (end 173.56 77.87) (width 0.5) (layer "F.Cu") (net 1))
 (segment (start 176.2 89.84) (end 122.86 89.84) (width 0.5) (layer "F.Cu") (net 1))
 (segment (start 179.8 76.625) (end 179.8 77.54) (width 0.5) (layer "F.Cu") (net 1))
 (segment (start 178 76.625) (end 177.445 76.625) (width 0.5) (layer "F.Cu") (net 1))
 (segment (start 177.445 76.625) (end 176.2 77.87) (width 0.5) (layer "F.Cu") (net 1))
 (segment (start 179.8 77.54) (end 179.47 77.87) (width 0.5) (layer "F.Cu") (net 1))
 (segment (start 178.74 73.87) (end 176.2 73.87) (width 0.5) (layer "F.Cu") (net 45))
 (segment (start 183.09 73.87) (end 183.82 74.6) (width 0.5) (layer "F.Cu") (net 45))
 (segment (start 176.2 73.87) (end 173.66 73.87) (width 0.5) (layer "F.Cu") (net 45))
 (segment (start 183.09 73.87) (end 178.74 73.87) (width 0.5) (layer "F.Cu") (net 45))
 (segment (start 122.225 93.015) (end 122.225 98.095) (width 0.5) (layer "F.Cu") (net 45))
 (segment (start 179.8 75.075) (end 179.8 74.93) (width 0.5) (layer "F.Cu") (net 45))
 (segment (start 179.8 74.93) (end 178.74 73.87) (width 0.5) (layer "F.Cu") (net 45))
 (segment (start 178 75.075) (end 177.405 75.075) (width 0.5) (layer "F.Cu") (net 45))
 (segment (start 183.82 74.6) (end 183.82 84.76) (width 0.5) (layer "F.Cu") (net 45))
 (segment (start 177.405 75.075) (end 176.2 73.87) (width 0.5) (layer "F.Cu") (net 45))
 (segment (start 176.2 92.38) (end 122.86 92.38) (width 0.5) (layer "F.Cu") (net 45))
 (segment (start 122.86 92.38) (end 122.225 93.015) (width 0.5) (layer "F.Cu") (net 45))
 (segment (start 183.82 84.76) (end 176.2 92.38) (width 0.5) (layer "F.Cu") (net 45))
 (segment (start 140.64 77.14) (end 140.64 82.22) (width 0.25) (layer "F.Cu") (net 56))
 (segment (start 143.91 73.87) (end 140.64 77.14) (width 0.25) (layer "F.Cu") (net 56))
 (segment (start 158.26 73.87) (end 143.91 73.87) (width 0.25) (layer "F.Cu") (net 56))
 (via (at 140.64 82.22) (size 0.6) (drill 0.4) (layers "F.Cu" "B.Cu") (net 56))
 (segment (start 140.64 82.22) (end 141.18 82.76) (width 0.25) (layer "B.Cu") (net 56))
 (segment (start 141.18 82.76) (end 141.18 96.92) (width 0.25) (layer "B.Cu") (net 56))
 (segment (start 141.18 96.92) (end 140.005 98.095) (width 0.25) (layer "B.Cu") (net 56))
 (segment (start 153.53 71.87) (end 153.34 72.06) (width 0.25) (layer "F.Cu") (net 60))
 (segment (start 153.34 72.06) (end 150.8 72.06) (width 0.25) (layer "F.Cu") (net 60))
 (segment (start 158.26 71.87) (end 153.53 71.87) (width 0.25) (layer "F.Cu") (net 60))
 (via (at 150.8 72.06) (size 0.6) (drill 0.4) (layers "F.Cu" "B.Cu") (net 60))
 (segment (start 146.26 96.92) (end 145.085 98.095) (width 0.25) (layer "B.Cu") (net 60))
 (segment (start 146.26 74.06) (end 146.26 96.92) (width 0.25) (layer "B.Cu") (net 60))
 (segment (start 150.8 72.06) (end 148.26 72.06) (width 0.25) (layer "B.Cu") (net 60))
 (segment (start 148.26 72.06) (end 146.26 74.06) (width 0.25) (layer "B.Cu") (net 60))
 (segment (start 158.26 69.87) (end 153.69 69.87) (width 0.25) (layer "F.Cu") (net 61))
 (segment (start 153.34 69.52) (end 150.8 69.52) (width 0.25) (layer "F.Cu") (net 61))
 (segment (start 153.69 69.87) (end 153.34 69.52) (width 0.25) (layer "F.Cu") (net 61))
 (via (at 150.8 69.52) (size 0.6) (drill 0.4) (layers "F.Cu" "B.Cu") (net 61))
 (segment (start 143.18 72.06) (end 143.18 93.65) (width 0.25) (layer "B.Cu") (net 61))
 (segment (start 143.18 93.65) (end 145.085 95.555) (width 0.25) (layer "B.Cu") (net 61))
 (segment (start 150.8 69.52) (end 145.72 69.52) (width 0.25) (layer "B.Cu") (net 61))
 (segment (start 145.72 69.52) (end 143.18 72.06) (width 0.25) (layer "B.Cu") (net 61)))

